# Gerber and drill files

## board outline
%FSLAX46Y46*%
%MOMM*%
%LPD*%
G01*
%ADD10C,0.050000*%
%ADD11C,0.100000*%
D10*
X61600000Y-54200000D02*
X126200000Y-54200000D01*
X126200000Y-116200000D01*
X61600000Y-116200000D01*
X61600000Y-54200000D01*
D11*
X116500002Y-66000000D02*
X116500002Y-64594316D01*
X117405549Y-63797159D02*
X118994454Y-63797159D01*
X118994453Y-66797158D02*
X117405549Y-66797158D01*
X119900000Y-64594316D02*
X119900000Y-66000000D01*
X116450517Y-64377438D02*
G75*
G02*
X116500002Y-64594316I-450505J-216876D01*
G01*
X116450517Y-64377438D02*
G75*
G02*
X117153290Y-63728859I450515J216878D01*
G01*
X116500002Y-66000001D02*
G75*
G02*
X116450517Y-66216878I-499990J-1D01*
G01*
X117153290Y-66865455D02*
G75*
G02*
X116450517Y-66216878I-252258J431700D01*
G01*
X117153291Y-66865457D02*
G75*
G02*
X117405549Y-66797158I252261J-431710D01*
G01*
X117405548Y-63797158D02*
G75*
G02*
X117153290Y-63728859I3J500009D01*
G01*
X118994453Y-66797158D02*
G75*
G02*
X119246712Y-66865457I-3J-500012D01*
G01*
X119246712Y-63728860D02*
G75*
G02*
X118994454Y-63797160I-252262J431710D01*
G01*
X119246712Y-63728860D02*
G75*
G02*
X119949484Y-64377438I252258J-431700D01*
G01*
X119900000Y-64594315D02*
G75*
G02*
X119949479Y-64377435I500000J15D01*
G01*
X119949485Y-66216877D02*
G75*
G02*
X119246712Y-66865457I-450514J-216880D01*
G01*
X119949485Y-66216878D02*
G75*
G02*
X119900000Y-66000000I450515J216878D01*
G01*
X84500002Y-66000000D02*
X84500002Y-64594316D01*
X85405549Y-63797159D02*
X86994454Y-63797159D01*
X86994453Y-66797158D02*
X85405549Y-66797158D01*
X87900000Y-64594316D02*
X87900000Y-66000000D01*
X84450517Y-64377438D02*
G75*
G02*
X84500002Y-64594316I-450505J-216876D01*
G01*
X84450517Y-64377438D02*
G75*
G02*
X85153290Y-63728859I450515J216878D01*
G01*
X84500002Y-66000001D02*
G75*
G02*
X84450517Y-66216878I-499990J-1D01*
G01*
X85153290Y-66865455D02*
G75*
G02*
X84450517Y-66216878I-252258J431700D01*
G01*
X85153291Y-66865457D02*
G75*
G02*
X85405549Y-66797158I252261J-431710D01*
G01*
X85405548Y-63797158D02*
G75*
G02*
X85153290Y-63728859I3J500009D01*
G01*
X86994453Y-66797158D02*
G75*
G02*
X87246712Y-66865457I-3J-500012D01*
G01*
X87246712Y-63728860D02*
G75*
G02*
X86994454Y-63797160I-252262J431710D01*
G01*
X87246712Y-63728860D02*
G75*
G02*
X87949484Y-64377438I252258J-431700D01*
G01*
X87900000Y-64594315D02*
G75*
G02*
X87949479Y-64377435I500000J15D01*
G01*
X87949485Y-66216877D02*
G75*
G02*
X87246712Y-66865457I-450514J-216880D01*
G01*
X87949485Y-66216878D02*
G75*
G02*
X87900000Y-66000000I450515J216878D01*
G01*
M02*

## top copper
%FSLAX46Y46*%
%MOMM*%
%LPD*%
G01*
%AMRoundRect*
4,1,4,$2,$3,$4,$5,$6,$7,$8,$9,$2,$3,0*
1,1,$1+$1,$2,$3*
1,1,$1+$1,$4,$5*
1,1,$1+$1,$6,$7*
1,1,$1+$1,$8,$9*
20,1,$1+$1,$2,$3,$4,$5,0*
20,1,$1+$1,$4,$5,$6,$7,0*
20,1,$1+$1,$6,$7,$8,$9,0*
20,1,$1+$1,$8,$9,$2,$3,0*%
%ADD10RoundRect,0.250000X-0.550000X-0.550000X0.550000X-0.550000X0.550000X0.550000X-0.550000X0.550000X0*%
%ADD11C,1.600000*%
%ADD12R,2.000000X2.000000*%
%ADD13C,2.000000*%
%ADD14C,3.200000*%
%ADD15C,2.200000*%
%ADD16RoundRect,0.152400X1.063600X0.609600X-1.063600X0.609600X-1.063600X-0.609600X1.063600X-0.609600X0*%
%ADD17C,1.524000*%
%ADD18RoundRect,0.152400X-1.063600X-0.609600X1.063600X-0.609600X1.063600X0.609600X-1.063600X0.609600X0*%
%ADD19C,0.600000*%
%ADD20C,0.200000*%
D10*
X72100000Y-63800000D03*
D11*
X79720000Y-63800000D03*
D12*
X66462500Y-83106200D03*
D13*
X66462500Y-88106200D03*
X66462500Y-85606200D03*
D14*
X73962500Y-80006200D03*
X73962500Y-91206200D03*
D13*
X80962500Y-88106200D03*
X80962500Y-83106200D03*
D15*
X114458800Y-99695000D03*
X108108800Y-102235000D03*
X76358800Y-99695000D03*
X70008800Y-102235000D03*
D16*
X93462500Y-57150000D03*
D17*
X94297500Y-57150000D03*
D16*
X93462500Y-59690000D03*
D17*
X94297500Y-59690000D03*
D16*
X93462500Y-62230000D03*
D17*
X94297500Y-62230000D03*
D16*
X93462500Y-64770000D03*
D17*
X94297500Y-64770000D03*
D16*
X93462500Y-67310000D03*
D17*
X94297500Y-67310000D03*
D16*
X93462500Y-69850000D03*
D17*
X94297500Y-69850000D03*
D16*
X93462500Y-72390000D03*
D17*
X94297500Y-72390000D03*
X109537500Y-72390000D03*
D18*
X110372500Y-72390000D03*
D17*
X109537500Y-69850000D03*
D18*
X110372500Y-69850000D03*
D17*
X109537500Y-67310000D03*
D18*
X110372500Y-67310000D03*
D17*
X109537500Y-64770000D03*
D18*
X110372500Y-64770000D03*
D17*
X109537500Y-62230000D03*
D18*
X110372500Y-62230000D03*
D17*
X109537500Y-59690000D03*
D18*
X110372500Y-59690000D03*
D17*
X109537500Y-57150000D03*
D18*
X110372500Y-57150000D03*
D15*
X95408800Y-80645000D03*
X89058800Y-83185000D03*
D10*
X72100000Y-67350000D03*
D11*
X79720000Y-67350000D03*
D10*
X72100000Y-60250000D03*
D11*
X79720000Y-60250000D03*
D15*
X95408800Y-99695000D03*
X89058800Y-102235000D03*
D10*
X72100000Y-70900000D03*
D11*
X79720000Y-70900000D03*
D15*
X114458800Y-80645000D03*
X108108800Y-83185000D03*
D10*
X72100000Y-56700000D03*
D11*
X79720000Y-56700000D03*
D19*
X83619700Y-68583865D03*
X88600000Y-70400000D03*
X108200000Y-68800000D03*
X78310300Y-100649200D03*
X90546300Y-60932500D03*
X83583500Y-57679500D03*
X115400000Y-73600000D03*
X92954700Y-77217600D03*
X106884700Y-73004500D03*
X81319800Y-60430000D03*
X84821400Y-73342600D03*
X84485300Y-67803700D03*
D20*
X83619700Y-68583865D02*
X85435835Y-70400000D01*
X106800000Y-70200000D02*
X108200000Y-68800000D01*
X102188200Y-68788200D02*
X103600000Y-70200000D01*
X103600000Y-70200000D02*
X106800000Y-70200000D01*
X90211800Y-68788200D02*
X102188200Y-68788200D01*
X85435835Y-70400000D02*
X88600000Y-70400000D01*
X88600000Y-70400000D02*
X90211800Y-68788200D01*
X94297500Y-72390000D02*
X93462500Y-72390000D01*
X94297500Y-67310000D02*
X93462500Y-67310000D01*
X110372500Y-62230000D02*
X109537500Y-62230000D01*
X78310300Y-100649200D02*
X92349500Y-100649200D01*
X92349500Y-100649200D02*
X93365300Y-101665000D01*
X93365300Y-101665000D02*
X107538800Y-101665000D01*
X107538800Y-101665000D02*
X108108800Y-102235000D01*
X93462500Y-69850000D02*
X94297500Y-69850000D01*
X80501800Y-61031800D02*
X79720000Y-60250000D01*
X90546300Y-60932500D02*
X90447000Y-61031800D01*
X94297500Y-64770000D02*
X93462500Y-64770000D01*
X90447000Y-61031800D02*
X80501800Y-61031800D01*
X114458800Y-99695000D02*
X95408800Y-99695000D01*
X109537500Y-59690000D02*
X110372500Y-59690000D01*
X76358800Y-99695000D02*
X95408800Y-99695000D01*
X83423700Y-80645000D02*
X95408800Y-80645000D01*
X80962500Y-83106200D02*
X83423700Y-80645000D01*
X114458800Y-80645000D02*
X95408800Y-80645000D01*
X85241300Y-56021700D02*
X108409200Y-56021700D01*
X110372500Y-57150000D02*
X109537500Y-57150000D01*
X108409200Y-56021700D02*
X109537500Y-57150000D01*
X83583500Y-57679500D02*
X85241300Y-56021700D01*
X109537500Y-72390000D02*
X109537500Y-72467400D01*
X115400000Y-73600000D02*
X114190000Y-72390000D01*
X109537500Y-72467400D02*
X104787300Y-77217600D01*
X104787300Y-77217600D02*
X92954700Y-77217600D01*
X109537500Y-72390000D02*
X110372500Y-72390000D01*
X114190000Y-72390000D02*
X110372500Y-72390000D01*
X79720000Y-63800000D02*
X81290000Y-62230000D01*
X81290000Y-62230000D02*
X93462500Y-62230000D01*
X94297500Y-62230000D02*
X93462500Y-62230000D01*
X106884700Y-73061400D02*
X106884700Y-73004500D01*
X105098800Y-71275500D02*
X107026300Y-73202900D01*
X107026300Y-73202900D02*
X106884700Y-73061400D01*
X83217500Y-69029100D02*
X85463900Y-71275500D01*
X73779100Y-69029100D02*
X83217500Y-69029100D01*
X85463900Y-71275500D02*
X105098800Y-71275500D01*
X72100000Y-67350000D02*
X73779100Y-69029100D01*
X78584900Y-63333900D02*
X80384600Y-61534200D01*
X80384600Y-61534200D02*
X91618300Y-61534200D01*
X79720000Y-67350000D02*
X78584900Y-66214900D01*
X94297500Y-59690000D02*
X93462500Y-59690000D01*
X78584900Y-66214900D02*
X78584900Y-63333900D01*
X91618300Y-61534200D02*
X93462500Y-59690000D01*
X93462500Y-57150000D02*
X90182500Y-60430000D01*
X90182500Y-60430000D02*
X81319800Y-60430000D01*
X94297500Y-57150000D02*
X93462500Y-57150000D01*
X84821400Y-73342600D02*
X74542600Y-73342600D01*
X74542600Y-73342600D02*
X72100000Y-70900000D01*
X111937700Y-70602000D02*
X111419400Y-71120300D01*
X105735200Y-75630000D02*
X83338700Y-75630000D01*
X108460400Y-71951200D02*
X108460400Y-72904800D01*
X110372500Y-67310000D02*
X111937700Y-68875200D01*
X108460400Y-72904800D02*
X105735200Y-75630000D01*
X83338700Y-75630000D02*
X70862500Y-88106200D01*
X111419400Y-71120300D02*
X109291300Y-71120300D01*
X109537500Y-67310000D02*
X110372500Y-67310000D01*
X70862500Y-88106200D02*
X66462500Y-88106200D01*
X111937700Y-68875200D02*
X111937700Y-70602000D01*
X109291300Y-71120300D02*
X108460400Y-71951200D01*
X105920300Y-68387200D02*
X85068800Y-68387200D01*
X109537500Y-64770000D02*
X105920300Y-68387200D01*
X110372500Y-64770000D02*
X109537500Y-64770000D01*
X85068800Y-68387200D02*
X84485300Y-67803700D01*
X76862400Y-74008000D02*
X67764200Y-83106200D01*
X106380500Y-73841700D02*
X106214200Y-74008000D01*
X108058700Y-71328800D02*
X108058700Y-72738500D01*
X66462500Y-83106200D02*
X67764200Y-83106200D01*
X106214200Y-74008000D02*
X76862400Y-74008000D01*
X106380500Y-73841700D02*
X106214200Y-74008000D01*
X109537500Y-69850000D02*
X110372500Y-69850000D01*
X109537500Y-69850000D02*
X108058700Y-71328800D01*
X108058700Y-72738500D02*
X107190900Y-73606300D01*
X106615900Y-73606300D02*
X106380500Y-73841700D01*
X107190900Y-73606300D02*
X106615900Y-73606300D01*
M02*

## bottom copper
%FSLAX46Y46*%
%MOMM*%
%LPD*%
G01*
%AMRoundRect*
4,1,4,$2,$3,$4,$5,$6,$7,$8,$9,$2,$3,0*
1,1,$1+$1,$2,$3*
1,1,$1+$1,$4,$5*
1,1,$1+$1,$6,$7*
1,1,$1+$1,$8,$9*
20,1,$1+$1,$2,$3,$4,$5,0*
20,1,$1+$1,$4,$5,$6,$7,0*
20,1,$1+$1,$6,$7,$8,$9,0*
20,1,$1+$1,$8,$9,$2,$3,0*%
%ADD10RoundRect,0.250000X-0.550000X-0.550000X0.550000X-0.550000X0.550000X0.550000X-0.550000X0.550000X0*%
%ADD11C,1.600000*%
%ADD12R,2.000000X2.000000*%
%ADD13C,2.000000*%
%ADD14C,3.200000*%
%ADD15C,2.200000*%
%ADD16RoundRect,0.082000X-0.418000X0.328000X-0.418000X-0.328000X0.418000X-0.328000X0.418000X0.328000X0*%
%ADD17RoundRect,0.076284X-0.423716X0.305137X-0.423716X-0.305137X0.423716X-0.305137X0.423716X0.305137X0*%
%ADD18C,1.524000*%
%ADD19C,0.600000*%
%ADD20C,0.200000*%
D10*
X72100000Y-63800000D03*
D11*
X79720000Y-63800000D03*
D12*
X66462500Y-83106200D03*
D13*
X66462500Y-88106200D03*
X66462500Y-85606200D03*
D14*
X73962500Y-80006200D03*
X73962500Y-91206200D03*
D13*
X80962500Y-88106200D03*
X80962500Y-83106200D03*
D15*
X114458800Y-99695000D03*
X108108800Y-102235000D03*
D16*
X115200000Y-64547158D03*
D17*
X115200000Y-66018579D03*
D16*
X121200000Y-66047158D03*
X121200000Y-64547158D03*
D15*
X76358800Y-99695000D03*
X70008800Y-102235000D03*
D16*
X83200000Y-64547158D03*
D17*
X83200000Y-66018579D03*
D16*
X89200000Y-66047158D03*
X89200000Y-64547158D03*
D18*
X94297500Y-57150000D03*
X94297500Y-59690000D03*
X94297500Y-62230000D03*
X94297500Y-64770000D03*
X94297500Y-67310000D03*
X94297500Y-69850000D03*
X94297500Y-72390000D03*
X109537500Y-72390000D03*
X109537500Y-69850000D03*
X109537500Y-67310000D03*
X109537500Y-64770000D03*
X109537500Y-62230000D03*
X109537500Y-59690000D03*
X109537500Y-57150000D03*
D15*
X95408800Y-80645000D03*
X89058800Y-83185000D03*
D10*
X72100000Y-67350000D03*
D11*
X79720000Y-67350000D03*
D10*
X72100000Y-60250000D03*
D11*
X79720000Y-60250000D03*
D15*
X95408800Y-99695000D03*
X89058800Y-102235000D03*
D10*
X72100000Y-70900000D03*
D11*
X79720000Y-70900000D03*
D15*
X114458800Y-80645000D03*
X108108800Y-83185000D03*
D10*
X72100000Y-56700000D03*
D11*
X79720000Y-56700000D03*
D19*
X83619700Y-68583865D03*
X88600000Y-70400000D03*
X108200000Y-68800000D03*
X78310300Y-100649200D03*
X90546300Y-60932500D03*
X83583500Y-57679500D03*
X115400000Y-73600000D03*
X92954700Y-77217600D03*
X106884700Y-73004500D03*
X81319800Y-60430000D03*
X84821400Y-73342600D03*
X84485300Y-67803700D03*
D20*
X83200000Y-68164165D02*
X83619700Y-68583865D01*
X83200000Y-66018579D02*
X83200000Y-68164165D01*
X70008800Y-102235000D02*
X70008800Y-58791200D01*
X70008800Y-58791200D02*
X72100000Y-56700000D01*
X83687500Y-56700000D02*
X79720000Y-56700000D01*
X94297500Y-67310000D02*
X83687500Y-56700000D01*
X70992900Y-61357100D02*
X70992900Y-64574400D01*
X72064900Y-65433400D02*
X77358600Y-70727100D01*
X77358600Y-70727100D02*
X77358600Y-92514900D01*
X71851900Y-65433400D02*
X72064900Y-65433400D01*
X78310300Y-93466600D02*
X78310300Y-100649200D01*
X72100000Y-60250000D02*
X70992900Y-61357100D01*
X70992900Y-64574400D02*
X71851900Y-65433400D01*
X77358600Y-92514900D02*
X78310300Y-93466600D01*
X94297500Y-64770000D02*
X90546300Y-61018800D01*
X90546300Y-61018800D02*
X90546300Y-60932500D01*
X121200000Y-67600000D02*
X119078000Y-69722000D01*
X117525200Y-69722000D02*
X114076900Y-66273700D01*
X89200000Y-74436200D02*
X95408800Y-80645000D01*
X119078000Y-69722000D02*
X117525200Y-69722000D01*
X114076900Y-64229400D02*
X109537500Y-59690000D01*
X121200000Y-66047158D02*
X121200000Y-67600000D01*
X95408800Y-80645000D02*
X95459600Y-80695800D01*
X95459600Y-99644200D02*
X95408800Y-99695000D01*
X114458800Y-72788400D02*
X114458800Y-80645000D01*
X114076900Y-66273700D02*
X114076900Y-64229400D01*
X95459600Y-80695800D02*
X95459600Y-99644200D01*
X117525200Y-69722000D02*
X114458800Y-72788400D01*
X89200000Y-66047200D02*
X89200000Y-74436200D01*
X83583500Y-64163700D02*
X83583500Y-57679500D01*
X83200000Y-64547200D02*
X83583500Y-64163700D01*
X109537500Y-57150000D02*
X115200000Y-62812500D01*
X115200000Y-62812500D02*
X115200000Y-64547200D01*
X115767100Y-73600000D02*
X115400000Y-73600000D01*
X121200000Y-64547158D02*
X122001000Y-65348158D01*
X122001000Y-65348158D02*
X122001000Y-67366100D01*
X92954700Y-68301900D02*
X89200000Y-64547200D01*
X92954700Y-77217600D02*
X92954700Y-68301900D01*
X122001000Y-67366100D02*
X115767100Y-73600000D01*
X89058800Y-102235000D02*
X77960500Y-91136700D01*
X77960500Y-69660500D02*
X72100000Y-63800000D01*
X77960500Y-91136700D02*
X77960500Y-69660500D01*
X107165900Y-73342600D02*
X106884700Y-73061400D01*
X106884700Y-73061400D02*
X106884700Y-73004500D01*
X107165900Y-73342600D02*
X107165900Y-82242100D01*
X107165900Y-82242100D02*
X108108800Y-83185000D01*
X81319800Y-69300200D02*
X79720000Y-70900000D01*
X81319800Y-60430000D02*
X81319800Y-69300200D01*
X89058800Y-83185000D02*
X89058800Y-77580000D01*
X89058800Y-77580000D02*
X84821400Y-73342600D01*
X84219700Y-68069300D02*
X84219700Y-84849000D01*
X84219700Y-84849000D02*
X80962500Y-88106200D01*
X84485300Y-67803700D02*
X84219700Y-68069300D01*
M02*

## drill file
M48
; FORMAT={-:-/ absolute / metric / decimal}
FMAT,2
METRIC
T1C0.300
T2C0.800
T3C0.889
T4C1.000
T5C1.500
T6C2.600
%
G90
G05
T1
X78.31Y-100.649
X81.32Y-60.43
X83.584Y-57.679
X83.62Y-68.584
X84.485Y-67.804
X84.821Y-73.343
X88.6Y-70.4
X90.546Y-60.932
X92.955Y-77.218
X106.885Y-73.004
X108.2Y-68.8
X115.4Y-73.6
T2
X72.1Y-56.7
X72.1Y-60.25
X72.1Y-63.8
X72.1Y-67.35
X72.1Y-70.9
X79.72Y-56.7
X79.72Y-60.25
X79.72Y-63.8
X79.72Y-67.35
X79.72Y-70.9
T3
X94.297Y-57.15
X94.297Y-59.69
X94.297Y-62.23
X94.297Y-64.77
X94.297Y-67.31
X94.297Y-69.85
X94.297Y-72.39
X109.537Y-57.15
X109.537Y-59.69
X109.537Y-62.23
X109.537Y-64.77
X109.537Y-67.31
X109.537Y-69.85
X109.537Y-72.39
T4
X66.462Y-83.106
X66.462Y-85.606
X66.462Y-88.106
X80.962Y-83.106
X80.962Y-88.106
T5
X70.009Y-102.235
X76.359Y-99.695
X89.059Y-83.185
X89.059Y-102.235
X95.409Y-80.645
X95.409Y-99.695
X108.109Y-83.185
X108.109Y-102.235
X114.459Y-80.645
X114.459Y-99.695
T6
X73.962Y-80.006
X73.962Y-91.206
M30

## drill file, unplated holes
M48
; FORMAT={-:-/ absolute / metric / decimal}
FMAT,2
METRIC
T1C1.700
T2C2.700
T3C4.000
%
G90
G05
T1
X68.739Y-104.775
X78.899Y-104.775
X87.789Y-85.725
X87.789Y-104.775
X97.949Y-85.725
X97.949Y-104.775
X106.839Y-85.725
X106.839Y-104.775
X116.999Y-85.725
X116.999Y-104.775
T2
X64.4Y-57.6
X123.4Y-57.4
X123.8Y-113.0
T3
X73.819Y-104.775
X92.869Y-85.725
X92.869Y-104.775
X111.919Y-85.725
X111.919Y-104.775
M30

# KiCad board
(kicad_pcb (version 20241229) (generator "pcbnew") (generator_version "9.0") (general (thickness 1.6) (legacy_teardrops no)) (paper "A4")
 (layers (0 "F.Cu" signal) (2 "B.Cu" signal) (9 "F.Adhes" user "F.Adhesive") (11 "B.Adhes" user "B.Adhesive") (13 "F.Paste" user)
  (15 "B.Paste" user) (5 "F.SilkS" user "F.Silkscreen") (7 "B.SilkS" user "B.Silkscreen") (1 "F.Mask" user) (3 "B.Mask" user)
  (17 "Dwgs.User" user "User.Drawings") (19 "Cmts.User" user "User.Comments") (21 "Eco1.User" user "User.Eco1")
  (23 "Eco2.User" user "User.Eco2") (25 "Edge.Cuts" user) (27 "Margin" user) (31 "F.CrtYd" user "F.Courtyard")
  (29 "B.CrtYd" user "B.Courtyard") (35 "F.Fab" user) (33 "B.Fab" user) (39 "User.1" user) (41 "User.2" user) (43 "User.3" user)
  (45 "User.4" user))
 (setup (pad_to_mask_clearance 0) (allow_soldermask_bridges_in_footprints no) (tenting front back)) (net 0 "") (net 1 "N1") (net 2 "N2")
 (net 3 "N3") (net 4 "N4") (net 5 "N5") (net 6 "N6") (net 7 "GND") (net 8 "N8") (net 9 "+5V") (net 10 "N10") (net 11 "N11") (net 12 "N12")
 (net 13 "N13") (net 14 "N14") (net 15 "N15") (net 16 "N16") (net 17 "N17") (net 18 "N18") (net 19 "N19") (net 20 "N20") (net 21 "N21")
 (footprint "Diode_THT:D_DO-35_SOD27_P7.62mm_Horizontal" (layer "F.Cu") (at 72.1 63.8)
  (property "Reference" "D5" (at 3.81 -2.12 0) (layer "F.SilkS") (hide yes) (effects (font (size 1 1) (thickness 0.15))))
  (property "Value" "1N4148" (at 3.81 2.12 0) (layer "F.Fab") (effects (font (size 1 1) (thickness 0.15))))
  (pad "1" thru_hole roundrect (at 0 0) (size 1.6 1.6) (drill 0.8) (layers "*.Cu" "*.Mask") (remove_unused_layers no)
   (roundrect_rratio 0.15625) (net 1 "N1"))
  (pad "2" thru_hole circle (at 7.62 0) (size 1.6 1.6) (drill 0.8) (layers "*.Cu" "*.Mask") (remove_unused_layers no) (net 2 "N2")))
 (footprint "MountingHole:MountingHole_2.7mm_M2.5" (layer "F.Cu") (at 123.4 57.4)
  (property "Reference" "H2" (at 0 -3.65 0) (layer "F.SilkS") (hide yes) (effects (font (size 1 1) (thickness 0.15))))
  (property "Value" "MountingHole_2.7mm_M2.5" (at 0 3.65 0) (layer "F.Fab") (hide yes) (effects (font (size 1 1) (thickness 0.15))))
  (pad "" np_thru_hole circle (at 0 0) (size 2.7 2.7) (drill 2.7) (layers "*.Cu" "*.Mask")))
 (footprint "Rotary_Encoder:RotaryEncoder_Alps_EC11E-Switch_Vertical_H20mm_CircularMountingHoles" (layer "F.Cu") (at 66.4625 83.1062)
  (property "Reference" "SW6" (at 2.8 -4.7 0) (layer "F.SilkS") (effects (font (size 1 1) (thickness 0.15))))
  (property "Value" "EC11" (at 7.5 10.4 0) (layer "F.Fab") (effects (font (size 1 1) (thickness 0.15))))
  (pad "A" thru_hole rect (at 0 0) (size 2 2) (drill 1) (layers "*.Cu" "*.Mask") (remove_unused_layers no) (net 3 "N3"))
  (pad "B" thru_hole circle (at 0 5) (size 2 2) (drill 1) (layers "*.Cu" "*.Mask") (remove_unused_layers no) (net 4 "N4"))
  (pad "C" thru_hole circle (at 0 2.5) (size 2 2) (drill 1) (layers "*.Cu" "*.Mask") (remove_unused_layers no) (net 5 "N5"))
  (pad "MP" thru_hole circle (at 7.5 -3.1) (size 3.2 3.2) (drill 2.6) (layers "*.Cu" "*.Mask") (remove_unused_layers no))
  (pad "MP" thru_hole circle (at 7.5 8.1) (size 3.2 3.2) (drill 2.6) (layers "*.Cu" "*.Mask") (remove_unused_layers no))
  (pad "S1" thru_hole circle (at 14.5 5) (size 2 2) (drill 1) (layers "*.Cu" "*.Mask") (remove_unused_layers no) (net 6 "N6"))
  (pad "S2" thru_hole circle (at 14.5 0) (size 2 2) (drill 1) (layers "*.Cu" "*.Mask") (remove_unused_layers no) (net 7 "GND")))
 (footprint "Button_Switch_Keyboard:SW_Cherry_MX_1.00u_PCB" (layer "F.Cu") (at 114.4588 99.695)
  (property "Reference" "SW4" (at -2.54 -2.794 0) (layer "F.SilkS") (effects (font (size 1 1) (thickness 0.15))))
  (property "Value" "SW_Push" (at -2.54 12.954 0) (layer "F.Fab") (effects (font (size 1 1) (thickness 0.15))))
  (pad "" np_thru_hole circle (at -7.62 5.08) (size 1.7 1.7) (drill 1.7) (layers "*.Cu" "*.Mask"))
  (pad "" np_thru_hole circle (at -2.54 5.08) (size 4 4) (drill 4) (layers "*.Cu" "*.Mask"))
  (pad "" np_thru_hole circle (at 2.54 5.08) (size 1.7 1.7) (drill 1.7) (layers "*.Cu" "*.Mask"))
  (pad "1" thru_hole circle (at 0 0) (size 2.2 2.2) (drill 1.5) (layers "*.Cu" "*.Mask") (remove_unused_layers no) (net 7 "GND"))
  (pad "2" thru_hole circle (at -6.35 2.54) (size 2.2 2.2) (drill 1.5) (layers "*.Cu" "*.Mask") (remove_unused_layers no) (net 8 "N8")))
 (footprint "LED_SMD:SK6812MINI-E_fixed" (layer "F.Cu") (at 118.2 65.4)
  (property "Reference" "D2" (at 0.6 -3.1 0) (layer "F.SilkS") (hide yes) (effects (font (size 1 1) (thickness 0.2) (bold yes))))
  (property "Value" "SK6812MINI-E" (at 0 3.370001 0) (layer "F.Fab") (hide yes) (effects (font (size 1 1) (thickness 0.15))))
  (fp_line (start -1.699998 0.6) (end -1.699998 -0.805684) (stroke (width 0.1) (type solid)) (layer "Edge.Cuts"))
  (fp_line (start -0.794451 -1.602841) (end 0.794454 -1.602841) (stroke (width 0.1) (type solid)) (layer "Edge.Cuts"))
  (fp_line (start 0.794453 1.397158) (end -0.794451 1.397158) (stroke (width 0.1) (type solid)) (layer "Edge.Cuts"))
  (fp_line (start 1.7 -0.805684) (end 1.7 0.6) (stroke (width 0.1) (type solid)) (layer "Edge.Cuts"))
  (fp_arc (start -1.749483 -1.022562) (mid -1.712526 -0.91691) (end -1.699998 -0.805684) (stroke (width 0.1) (type solid))
   (layer "Edge.Cuts"))
  (fp_arc (start -1.749483 -1.022562) (mid -1.63807 -1.606877) (end -1.04671 -1.671141) (stroke (width 0.1) (type solid))
   (layer "Edge.Cuts"))
  (fp_arc (start -1.699998 0.600001) (mid -1.712526 0.711226) (end -1.749483 0.816878) (stroke (width 0.1) (type solid)) (layer "Edge.Cuts"))
  (fp_arc (start -1.04671 1.465455) (mid -1.638069 1.401192) (end -1.749483 0.816878) (stroke (width 0.1) (type solid)) (layer "Edge.Cuts"))
  (fp_arc (start -1.046709 1.465457) (mid -0.925121 1.414535) (end -0.794451 1.397158) (stroke (width 0.1) (type solid)) (layer "Edge.Cuts"))
  (fp_arc (start -0.794452 -1.602842) (mid -0.925122 -1.620219) (end -1.04671 -1.671141) (stroke (width 0.1) (type solid))
   (layer "Edge.Cuts"))
  (fp_arc (start 0.794453 1.397158) (mid 0.925124 1.414535) (end 1.046712 1.465457) (stroke (width 0.1) (type solid)) (layer "Edge.Cuts"))
  (fp_arc (start 1.046712 -1.67114) (mid 0.925124 -1.620218) (end 0.794454 -1.602841) (stroke (width 0.1) (type solid)) (layer "Edge.Cuts"))
  (fp_arc (start 1.046712 -1.67114) (mid 1.638072 -1.606876) (end 1.749485 -1.022562) (stroke (width 0.1) (type solid)) (layer "Edge.Cuts"))
  (fp_arc (start 1.7 -0.805685) (mid 1.712528 -0.91691) (end 1.749485 -1.022562) (stroke (width 0.1) (type solid)) (layer "Edge.Cuts"))
  (fp_arc (start 1.749485 0.816877) (mid 1.638073 1.401193) (end 1.046712 1.465457) (stroke (width 0.1) (type solid)) (layer "Edge.Cuts"))
  (fp_arc (start 1.749485 0.816878) (mid 1.712528 0.711226) (end 1.7 0.6) (stroke (width 0.1) (type solid)) (layer "Edge.Cuts"))
  (pad "1" smd roundrect (at -3 -0.852842 270) (size 0.82 1) (layers "B.Cu" "B.Mask" "B.Paste") (roundrect_rratio 0.1) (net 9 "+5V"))
  (pad "2" smd roundrect (at -3 0.618579 270) (size 0.762842 1) (layers "B.Cu" "B.Mask" "B.Paste") (roundrect_rratio 0.1) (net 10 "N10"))
  (pad "3" smd roundrect (at 3 0.647158 270) (size 0.82 1) (layers "B.Cu" "B.Mask" "B.Paste") (roundrect_rratio 0.1) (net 7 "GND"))
  (pad "4" smd roundrect (at 3 -0.852842 270) (size 0.82 1) (layers "B.Cu" "B.Mask" "B.Paste") (roundrect_rratio 0.1) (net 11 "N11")))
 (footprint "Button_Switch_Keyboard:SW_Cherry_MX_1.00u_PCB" (layer "F.Cu") (at 76.3588 99.695)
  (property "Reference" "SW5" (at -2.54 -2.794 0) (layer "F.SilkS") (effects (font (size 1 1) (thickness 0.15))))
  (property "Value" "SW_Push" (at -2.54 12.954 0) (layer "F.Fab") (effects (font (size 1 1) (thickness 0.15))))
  (pad "" np_thru_hole circle (at -7.62 5.08) (size 1.7 1.7) (drill 1.7) (layers "*.Cu" "*.Mask"))
  (pad "" np_thru_hole circle (at -2.54 5.08) (size 4 4) (drill 4) (layers "*.Cu" "*.Mask"))
  (pad "" np_thru_hole circle (at 2.54 5.08) (size 1.7 1.7) (drill 1.7) (layers "*.Cu" "*.Mask"))
  (pad "1" thru_hole circle (at 0 0) (size 2.2 2.2) (drill 1.5) (layers "*.Cu" "*.Mask") (remove_unused_layers no) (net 7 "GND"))
  (pad "2" thru_hole circle (at -6.35 2.54) (size 2.2 2.2) (drill 1.5) (layers "*.Cu" "*.Mask") (remove_unused_layers no) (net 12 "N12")))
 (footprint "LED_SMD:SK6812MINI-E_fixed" (layer "F.Cu") (at 86.2 65.4)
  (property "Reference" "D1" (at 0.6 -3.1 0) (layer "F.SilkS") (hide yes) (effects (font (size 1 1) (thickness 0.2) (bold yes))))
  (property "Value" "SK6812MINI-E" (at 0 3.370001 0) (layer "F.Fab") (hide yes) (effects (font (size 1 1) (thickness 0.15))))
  (fp_line (start -1.699998 0.6) (end -1.699998 -0.805684) (stroke (width 0.1) (type solid)) (layer "Edge.Cuts"))
  (fp_line (start -0.794451 -1.602841) (end 0.794454 -1.602841) (stroke (width 0.1) (type solid)) (layer "Edge.Cuts"))
  (fp_line (start 0.794453 1.397158) (end -0.794451 1.397158) (stroke (width 0.1) (type solid)) (layer "Edge.Cuts"))
  (fp_line (start 1.7 -0.805684) (end 1.7 0.6) (stroke (width 0.1) (type solid)) (layer "Edge.Cuts"))
  (fp_arc (start -1.749483 -1.022562) (mid -1.712526 -0.91691) (end -1.699998 -0.805684) (stroke (width 0.1) (type solid))
   (layer "Edge.Cuts"))
  (fp_arc (start -1.749483 -1.022562) (mid -1.63807 -1.606877) (end -1.04671 -1.671141) (stroke (width 0.1) (type solid))
   (layer "Edge.Cuts"))
  (fp_arc (start -1.699998 0.600001) (mid -1.712526 0.711226) (end -1.749483 0.816878) (stroke (width 0.1) (type solid)) (layer "Edge.Cuts"))
  (fp_arc (start -1.04671 1.465455) (mid -1.638069 1.401192) (end -1.749483 0.816878) (stroke (width 0.1) (type solid)) (layer "Edge.Cuts"))
  (fp_arc (start -1.046709 1.465457) (mid -0.925121 1.414535) (end -0.794451 1.397158) (stroke (width 0.1) (type solid)) (layer "Edge.Cuts"))
  (fp_arc (start -0.794452 -1.602842) (mid -0.925122 -1.620219) (end -1.04671 -1.671141) (stroke (width 0.1) (type solid))
   (layer "Edge.Cuts"))
  (fp_arc (start 0.794453 1.397158) (mid 0.925124 1.414535) (end 1.046712 1.465457) (stroke (width 0.1) (type solid)) (layer "Edge.Cuts"))
  (fp_arc (start 1.046712 -1.67114) (mid 0.925124 -1.620218) (end 0.794454 -1.602841) (stroke (width 0.1) (type solid)) (layer "Edge.Cuts"))
  (fp_arc (start 1.046712 -1.67114) (mid 1.638072 -1.606876) (end 1.749485 -1.022562) (stroke (width 0.1) (type solid)) (layer "Edge.Cuts"))
  (fp_arc (start 1.7 -0.805685) (mid 1.712528 -0.91691) (end 1.749485 -1.022562) (stroke (width 0.1) (type solid)) (layer "Edge.Cuts"))
  (fp_arc (start 1.749485 0.816877) (mid 1.638073 1.401193) (end 1.046712 1.465457) (stroke (width 0.1) (type solid)) (layer "Edge.Cuts"))
  (fp_arc (start 1.749485 0.816878) (mid 1.712528 0.711226) (end 1.7 0.6) (stroke (width 0.1) (type solid)) (layer "Edge.Cuts"))
  (pad "1" smd roundrect (at -3 -0.852842 270) (size 0.82 1) (layers "B.Cu" "B.Mask" "B.Paste") (roundrect_rratio 0.1) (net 9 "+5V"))
  (pad "2" smd roundrect (at -3 0.618579 270) (size 0.762842 1) (layers "B.Cu" "B.Mask" "B.Paste") (roundrect_rratio 0.1))
  (pad "3" smd roundrect (at 3 0.647158 270) (size 0.82 1) (layers "B.Cu" "B.Mask" "B.Paste") (roundrect_rratio 0.1) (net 7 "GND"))
  (pad "4" smd roundrect (at 3 -0.852842 270) (size 0.82 1) (layers "B.Cu" "B.Mask" "B.Paste") (roundrect_rratio 0.1) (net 11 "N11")))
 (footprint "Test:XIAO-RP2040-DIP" (layer "F.Cu") (at 101.9175 64.77)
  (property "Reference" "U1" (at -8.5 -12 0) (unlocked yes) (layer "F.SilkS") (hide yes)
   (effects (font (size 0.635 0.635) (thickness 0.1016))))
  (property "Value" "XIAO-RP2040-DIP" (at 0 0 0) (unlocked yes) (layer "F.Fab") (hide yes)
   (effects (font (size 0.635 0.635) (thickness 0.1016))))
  (pad "1" smd roundrect (at -8.455 -7.62 180) (size 2.432 1.524) (layers "F.Cu" "F.Mask") (roundrect_rratio 0.1) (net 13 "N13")
   (thermal_bridge_angle 45))
  (pad "1" thru_hole circle (at -7.62 -7.62 180) (size 1.524 1.524) (drill 0.889) (layers "*.Cu" "*.Mask") (remove_unused_layers no)
   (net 13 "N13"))
  (pad "2" smd roundrect (at -8.455 -5.08 180) (size 2.432 1.524) (layers "F.Cu" "F.Mask") (roundrect_rratio 0.1) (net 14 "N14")
   (thermal_bridge_angle 45))
  (pad "2" thru_hole circle (at -7.62 -5.08 180) (size 1.524 1.524) (drill 0.889) (layers "*.Cu" "*.Mask") (remove_unused_layers no)
   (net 14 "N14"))
  (pad "3" smd roundrect (at -8.455 -2.54 180) (size 2.432 1.524) (layers "F.Cu" "F.Mask") (roundrect_rratio 0.1) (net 2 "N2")
   (thermal_bridge_angle 45))
  (pad "3" thru_hole circle (at -7.62 -2.54 180) (size 1.524 1.524) (drill 0.889) (layers "*.Cu" "*.Mask") (remove_unused_layers no)
   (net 2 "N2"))
  (pad "4" smd roundrect (at -8.455 0 180) (size 2.432 1.524) (layers "F.Cu" "F.Mask") (roundrect_rratio 0.1) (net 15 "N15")
   (thermal_bridge_angle 45))
  (pad "4" thru_hole circle (at -7.62 0 180) (size 1.524 1.524) (drill 0.889) (layers "*.Cu" "*.Mask") (remove_unused_layers no)
   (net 15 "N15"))
  (pad "5" smd roundrect (at -8.455 2.54 180) (size 2.432 1.524) (layers "F.Cu" "F.Mask") (roundrect_rratio 0.1) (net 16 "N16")
   (thermal_bridge_angle 45))
  (pad "5" thru_hole circle (at -7.62 2.54 180) (size 1.524 1.524) (drill 0.889) (layers "*.Cu" "*.Mask") (remove_unused_layers no)
   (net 16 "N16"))
  (pad "6" smd roundrect (at -8.455 5.08 180) (size 2.432 1.524) (layers "F.Cu" "F.Mask") (roundrect_rratio 0.1) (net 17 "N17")
   (thermal_bridge_angle 45))
  (pad "6" thru_hole circle (at -7.62 5.08 180) (size 1.524 1.524) (drill 0.889) (layers "*.Cu" "*.Mask") (remove_unused_layers no)
   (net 17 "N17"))
  (pad "7" smd roundrect (at -8.455 7.62 180) (size 2.432 1.524) (layers "F.Cu" "F.Mask") (roundrect_rratio 0.1) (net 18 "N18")
   (thermal_bridge_angle 45))
  (pad "7" thru_hole circle (at -7.62 7.62 180) (size 1.524 1.524) (drill 0.889) (layers "*.Cu" "*.Mask") (remove_unused_layers no)
   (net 18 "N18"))
  (pad "8" thru_hole circle (at 7.62 7.62) (size 1.524 1.524) (drill 0.889) (layers "*.Cu" "*.Mask") (remove_unused_layers no)
   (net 11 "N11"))
  (pad "8" smd roundrect (at 8.455 7.62) (size 2.432 1.524) (layers "F.Cu" "F.Mask") (roundrect_rratio 0.1) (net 11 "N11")
   (thermal_bridge_angle 45))
  (pad "9" thru_hole circle (at 7.62 5.08) (size 1.524 1.524) (drill 0.889) (layers "*.Cu" "*.Mask") (remove_unused_layers no) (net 3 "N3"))
  (pad "9" smd roundrect (at 8.455 5.08) (size 2.432 1.524) (layers "F.Cu" "F.Mask") (roundrect_rratio 0.1) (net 3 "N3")
   (thermal_bridge_angle 45))
  (pad "10" thru_hole circle (at 7.62 2.54) (size 1.524 1.524) (drill 0.889) (layers "*.Cu" "*.Mask") (remove_unused_layers no) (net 4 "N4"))
  (pad "10" smd roundrect (at 8.455 2.54) (size 2.432 1.524) (layers "F.Cu" "F.Mask") (roundrect_rratio 0.1) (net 4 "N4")
   (thermal_bridge_angle 45))
  (pad "11" thru_hole circle (at 7.62 0) (size 1.524 1.524) (drill 0.889) (layers "*.Cu" "*.Mask") (remove_unused_layers no) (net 6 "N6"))
  (pad "11" smd roundrect (at 8.455 0) (size 2.432 1.524) (layers "F.Cu" "F.Mask") (roundrect_rratio 0.1) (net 6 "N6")
   (thermal_bridge_angle 45))
  (pad "12" thru_hole circle (at 7.62 -2.54) (size 1.524 1.524) (drill 0.889) (layers "*.Cu" "*.Mask") (remove_unused_layers no)
   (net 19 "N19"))
  (pad "12" smd roundrect (at 8.455 -2.54) (size 2.432 1.524) (layers "F.Cu" "F.Mask") (roundrect_rratio 0.1) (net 19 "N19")
   (thermal_bridge_angle 45))
  (pad "13" thru_hole circle (at 7.62 -5.08) (size 1.524 1.524) (drill 0.889) (layers "*.Cu" "*.Mask") (remove_unused_layers no)
   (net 7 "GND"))
  (pad "13" smd roundrect (at 8.455 -5.08) (size 2.432 1.524) (layers "F.Cu" "F.Mask") (roundrect_rratio 0.1) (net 7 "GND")
   (thermal_bridge_angle 45))
  (pad "14" thru_hole circle (at 7.62 -7.62) (size 1.524 1.524) (drill 0.889) (layers "*.Cu" "*.Mask") (remove_unused_layers no)
   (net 9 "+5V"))
  (pad "14" smd roundrect (at 8.455 -7.62) (size 2.432 1.524) (layers "F.Cu" "F.Mask") (roundrect_rratio 0.1) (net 9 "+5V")
   (thermal_bridge_angle 45)))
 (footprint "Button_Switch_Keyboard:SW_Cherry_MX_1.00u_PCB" (layer "F.Cu") (at 95.4088 80.645)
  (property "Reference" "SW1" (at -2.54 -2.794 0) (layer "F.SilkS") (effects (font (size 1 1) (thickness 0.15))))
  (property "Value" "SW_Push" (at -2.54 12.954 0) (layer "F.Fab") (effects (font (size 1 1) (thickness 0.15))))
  (pad "" np_thru_hole circle (at -7.62 5.08) (size 1.7 1.7) (drill 1.7) (layers "*.Cu" "*.Mask"))
  (pad "" np_thru_hole circle (at -2.54 5.08) (size 4 4) (drill 4) (layers "*.Cu" "*.Mask"))
  (pad "" np_thru_hole circle (at 2.54 5.08) (size 1.7 1.7) (drill 1.7) (layers "*.Cu" "*.Mask"))
  (pad "1" thru_hole circle (at 0 0) (size 2.2 2.2) (drill 1.5) (layers "*.Cu" "*.Mask") (remove_unused_layers no) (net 7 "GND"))
  (pad "2" thru_hole circle (at -6.35 2.54) (size 2.2 2.2) (drill 1.5) (layers "*.Cu" "*.Mask") (remove_unused_layers no) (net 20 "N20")))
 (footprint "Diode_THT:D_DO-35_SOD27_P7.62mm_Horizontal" (layer "F.Cu") (at 72.1 67.35)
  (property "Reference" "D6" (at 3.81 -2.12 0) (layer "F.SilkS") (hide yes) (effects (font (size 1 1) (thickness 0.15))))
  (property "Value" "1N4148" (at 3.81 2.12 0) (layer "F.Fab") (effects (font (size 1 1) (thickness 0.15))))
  (pad "1" thru_hole roundrect (at 0 0) (size 1.6 1.6) (drill 0.8) (layers "*.Cu" "*.Mask") (remove_unused_layers no)
   (roundrect_rratio 0.15625) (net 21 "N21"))
  (pad "2" thru_hole circle (at 7.62 0) (size 1.6 1.6) (drill 0.8) (layers "*.Cu" "*.Mask") (remove_unused_layers no) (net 14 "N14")))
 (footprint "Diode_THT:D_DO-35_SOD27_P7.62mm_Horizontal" (layer "F.Cu") (at 72.1 60.25)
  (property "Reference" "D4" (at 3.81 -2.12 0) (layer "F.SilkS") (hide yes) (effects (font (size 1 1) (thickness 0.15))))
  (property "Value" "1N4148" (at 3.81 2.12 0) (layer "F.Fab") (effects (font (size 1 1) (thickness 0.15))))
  (pad "1" thru_hole roundrect (at 0 0) (size 1.6 1.6) (drill 0.8) (layers "*.Cu" "*.Mask") (remove_unused_layers no)
   (roundrect_rratio 0.15625) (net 8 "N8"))
  (pad "2" thru_hole circle (at 7.62 0) (size 1.6 1.6) (drill 0.8) (layers "*.Cu" "*.Mask") (remove_unused_layers no) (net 15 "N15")))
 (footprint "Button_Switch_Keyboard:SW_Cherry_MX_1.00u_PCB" (layer "F.Cu") (at 95.4088 99.695)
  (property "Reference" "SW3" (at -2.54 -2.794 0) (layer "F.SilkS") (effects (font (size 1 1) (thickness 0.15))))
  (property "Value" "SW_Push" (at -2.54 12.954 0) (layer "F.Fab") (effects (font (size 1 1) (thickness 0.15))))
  (pad "" np_thru_hole circle (at -7.62 5.08) (size 1.7 1.7) (drill 1.7) (layers "*.Cu" "*.Mask"))
  (pad "" np_thru_hole circle (at -2.54 5.08) (size 4 4) (drill 4) (layers "*.Cu" "*.Mask"))
  (pad "" np_thru_hole circle (at 2.54 5.08) (size 1.7 1.7) (drill 1.7) (layers "*.Cu" "*.Mask"))
  (pad "1" thru_hole circle (at 0 0) (size 2.2 2.2) (drill 1.5) (layers "*.Cu" "*.Mask") (remove_unused_layers no) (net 7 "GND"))
  (pad "2" thru_hole circle (at -6.35 2.54) (size 2.2 2.2) (drill 1.5) (layers "*.Cu" "*.Mask") (remove_unused_layers no) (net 1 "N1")))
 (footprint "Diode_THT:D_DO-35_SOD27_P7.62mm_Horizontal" (layer "F.Cu") (at 72.1 70.9)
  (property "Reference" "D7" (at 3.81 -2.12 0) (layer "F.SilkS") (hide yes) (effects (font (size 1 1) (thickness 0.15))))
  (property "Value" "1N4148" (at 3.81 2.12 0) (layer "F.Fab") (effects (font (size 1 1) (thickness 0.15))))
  (pad "1" thru_hole roundrect (at 0 0) (size 1.6 1.6) (drill 0.8) (layers "*.Cu" "*.Mask") (remove_unused_layers no)
   (roundrect_rratio 0.15625) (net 20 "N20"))
  (pad "2" thru_hole circle (at 7.62 0) (size 1.6 1.6) (drill 0.8) (layers "*.Cu" "*.Mask") (remove_unused_layers no) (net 13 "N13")))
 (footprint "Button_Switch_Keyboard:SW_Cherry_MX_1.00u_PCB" (layer "F.Cu") (at 114.4588 80.645)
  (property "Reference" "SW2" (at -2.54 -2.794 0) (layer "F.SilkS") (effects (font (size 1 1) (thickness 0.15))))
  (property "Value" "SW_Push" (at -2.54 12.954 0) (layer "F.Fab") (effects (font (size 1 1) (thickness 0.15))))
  (pad "" np_thru_hole circle (at -7.62 5.08) (size 1.7 1.7) (drill 1.7) (layers "*.Cu" "*.Mask"))
  (pad "" np_thru_hole circle (at -2.54 5.08) (size 4 4) (drill 4) (layers "*.Cu" "*.Mask"))
  (pad "" np_thru_hole circle (at 2.54 5.08) (size 1.7 1.7) (drill 1.7) (layers "*.Cu" "*.Mask"))
  (pad "1" thru_hole circle (at 0 0) (size 2.2 2.2) (drill 1.5) (layers "*.Cu" "*.Mask") (remove_unused_layers no) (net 7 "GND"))
  (pad "2" thru_hole circle (at -6.35 2.54) (size 2.2 2.2) (drill 1.5) (layers "*.Cu" "*.Mask") (remove_unused_layers no) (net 21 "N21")))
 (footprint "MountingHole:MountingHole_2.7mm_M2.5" (layer "F.Cu") (at 64.4 57.6)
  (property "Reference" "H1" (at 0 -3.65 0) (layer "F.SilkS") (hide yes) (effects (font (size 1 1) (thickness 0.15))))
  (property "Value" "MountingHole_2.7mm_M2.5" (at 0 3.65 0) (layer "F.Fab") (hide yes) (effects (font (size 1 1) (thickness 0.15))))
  (pad "" np_thru_hole circle (at 0 0) (size 2.7 2.7) (drill 2.7) (layers "*.Cu" "*.Mask")))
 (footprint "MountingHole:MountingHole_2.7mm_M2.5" (layer "F.Cu") (at 123.8 113)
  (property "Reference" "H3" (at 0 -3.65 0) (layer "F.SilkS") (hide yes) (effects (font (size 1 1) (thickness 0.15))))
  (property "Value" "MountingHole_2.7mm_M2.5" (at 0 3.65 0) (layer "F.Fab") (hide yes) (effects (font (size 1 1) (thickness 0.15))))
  (pad "" np_thru_hole circle (at 0 0) (size 2.7 2.7) (drill 2.7) (layers "*.Cu" "*.Mask")))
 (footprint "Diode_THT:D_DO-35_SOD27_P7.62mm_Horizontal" (layer "F.Cu") (at 72.1 56.7)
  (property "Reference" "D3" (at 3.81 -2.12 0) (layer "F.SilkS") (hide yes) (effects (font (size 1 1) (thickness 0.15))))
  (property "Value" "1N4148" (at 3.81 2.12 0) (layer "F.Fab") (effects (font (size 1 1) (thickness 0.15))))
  (pad "1" thru_hole roundrect (at 0 0) (size 1.6 1.6) (drill 0.8) (layers "*.Cu" "*.Mask") (remove_unused_layers no)
   (roundrect_rratio 0.15625) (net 12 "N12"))
  (pad "2" thru_hole circle (at 7.62 0) (size 1.6 1.6) (drill 0.8) (layers "*.Cu" "*.Mask") (remove_unused_layers no) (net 16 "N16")))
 (gr_rect (start 61.6 54.2) (end 126.2 116.2) (stroke (width 0.05) (type default)) (fill no) (layer "Edge.Cuts"))
 (segment (start 83.6197 68.583865) (end 85.435835 70.4) (width 0.2) (layer "F.Cu") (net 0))
 (segment (start 106.8 70.2) (end 108.2 68.8) (width 0.2) (layer "F.Cu") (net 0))
 (segment (start 102.1882 68.7882) (end 103.6 70.2) (width 0.2) (layer "F.Cu") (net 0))
 (segment (start 103.6 70.2) (end 106.8 70.2) (width 0.2) (layer "F.Cu") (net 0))
 (segment (start 90.2118 68.7882) (end 102.1882 68.7882) (width 0.2) (layer "F.Cu") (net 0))
 (segment (start 85.435835 70.4) (end 88.6 70.4) (width 0.2) (layer "F.Cu") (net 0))
 (segment (start 88.6 70.4) (end 90.2118 68.7882) (width 0.2) (layer "F.Cu") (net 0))
 (via (at 83.6197 68.583865) (size 0.6) (drill 0.3) (layers "F.Cu" "B.Cu") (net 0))
 (via (at 88.6 70.4) (size 0.6) (drill 0.3) (layers "F.Cu" "B.Cu") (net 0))
 (via (at 108.2 68.8) (size 0.6) (drill 0.3) (layers "F.Cu" "B.Cu") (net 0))
 (segment (start 83.2 68.164165) (end 83.6197 68.583865) (width 0.2) (layer "B.Cu") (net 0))
 (segment (start 83.2 66.018579) (end 83.2 68.164165) (width 0.2) (layer "B.Cu") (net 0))
 (segment (start 94.2975 72.39) (end 93.4625 72.39) (width 0.2) (layer "F.Cu") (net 18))
 (segment (start 70.0088 102.235) (end 70.0088 58.7912) (width 0.2) (layer "B.Cu") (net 12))
 (segment (start 70.0088 58.7912) (end 72.1 56.7) (width 0.2) (layer "B.Cu") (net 12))
 (segment (start 94.2975 67.31) (end 93.4625 67.31) (width 0.2) (layer "F.Cu") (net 16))
 (segment (start 83.6875 56.7) (end 79.72 56.7) (width 0.2) (layer "B.Cu") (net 16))
 (segment (start 94.2975 67.31) (end 83.6875 56.7) (width 0.2) (layer "B.Cu") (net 16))
 (segment (start 110.3725 62.23) (end 109.5375 62.23) (width 0.2) (layer "F.Cu") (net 19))
 (segment (start 78.3103 100.6492) (end 92.3495 100.6492) (width 0.2) (layer "F.Cu") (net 8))
 (segment (start 92.3495 100.6492) (end 93.3653 101.665) (width 0.2) (layer "F.Cu") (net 8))
 (segment (start 93.3653 101.665) (end 107.5388 101.665) (width 0.2) (layer "F.Cu") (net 8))
 (segment (start 107.5388 101.665) (end 108.1088 102.235) (width 0.2) (layer "F.Cu") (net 8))
 (via (at 78.3103 100.6492) (size 0.6) (drill 0.3) (layers "F.Cu" "B.Cu") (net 8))
 (segment (start 70.9929 61.3571) (end 70.9929 64.5744) (width 0.2) (layer "B.Cu") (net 8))
 (segment (start 72.0649 65.4334) (end 77.3586 70.7271) (width 0.2) (layer "B.Cu") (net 8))
 (segment (start 77.3586 70.7271) (end 77.3586 92.5149) (width 0.2) (layer "B.Cu") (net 8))
 (segment (start 71.8519 65.4334) (end 72.0649 65.4334) (width 0.2) (layer "B.Cu") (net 8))
 (segment (start 78.3103 93.4666) (end 78.3103 100.6492) (width 0.2) (layer "B.Cu") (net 8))
 (segment (start 72.1 60.25) (end 70.9929 61.3571) (width 0.2) (layer "B.Cu") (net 8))
 (segment (start 70.9929 64.5744) (end 71.8519 65.4334) (width 0.2) (layer "B.Cu") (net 8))
 (segment (start 77.3586 92.5149) (end 78.3103 93.4666) (width 0.2) (layer "B.Cu") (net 8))
 (segment (start 93.4625 69.85) (end 94.2975 69.85) (width 0.2) (layer "F.Cu") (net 17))
 (segment (start 80.5018 61.0318) (end 79.72 60.25) (width 0.2) (layer "F.Cu") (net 15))
 (segment (start 90.5463 60.9325) (end 90.447 61.0318) (width 0.2) (layer "F.Cu") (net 15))
 (segment (start 94.2975 64.77) (end 93.4625 64.77) (width 0.2) (layer "F.Cu") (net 15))
 (segment (start 90.447 61.0318) (end 80.5018 61.0318) (width 0.2) (layer "F.Cu") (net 15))
 (via (at 90.5463 60.9325) (size 0.6) (drill 0.3) (layers "F.Cu" "B.Cu") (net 15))
 (segment (start 94.2975 64.77) (end 90.5463 61.0188) (width 0.2) (layer "B.Cu") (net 15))
 (segment (start 90.5463 61.0188) (end 90.5463 60.9325) (width 0.2) (layer "B.Cu") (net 15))
 (segment (start 114.4588 99.695) (end 95.4088 99.695) (width 0.2) (layer "F.Cu") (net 7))
 (segment (start 109.5375 59.69) (end 110.3725 59.69) (width 0.2) (layer "F.Cu") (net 7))
 (segment (start 76.3588 99.695) (end 95.4088 99.695) (width 0.2) (layer "F.Cu") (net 7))
 (segment (start 83.4237 80.645) (end 95.4088 80.645) (width 0.2) (layer "F.Cu") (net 7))
 (segment (start 80.9625 83.1062) (end 83.4237 80.645) (width 0.2) (layer "F.Cu") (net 7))
 (segment (start 114.4588 80.645) (end 95.4088 80.645) (width 0.2) (layer "F.Cu") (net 7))
 (segment (start 121.2 67.6) (end 119.078 69.722) (width 0.2) (layer "B.Cu") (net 7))
 (segment (start 117.5252 69.722) (end 114.0769 66.2737) (width 0.2) (layer "B.Cu") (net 7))
 (segment (start 89.2 74.4362) (end 95.4088 80.645) (width 0.2) (layer "B.Cu") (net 7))
 (segment (start 119.078 69.722) (end 117.5252 69.722) (width 0.2) (layer "B.Cu") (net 7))
 (segment (start 114.0769 64.2294) (end 109.5375 59.69) (width 0.2) (layer "B.Cu") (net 7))
 (segment (start 121.2 66.047158) (end 121.2 67.6) (width 0.2) (layer "B.Cu") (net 7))
 (segment (start 95.4088 80.645) (end 95.4596 80.6958) (width 0.2) (layer "B.Cu") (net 7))
 (segment (start 95.4596 99.6442) (end 95.4088 99.695) (width 0.2) (layer "B.Cu") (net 7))
 (segment (start 114.4588 72.7884) (end 114.4588 80.645) (width 0.2) (layer "B.Cu") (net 7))
 (segment (start 114.0769 66.2737) (end 114.0769 64.2294) (width 0.2) (layer "B.Cu") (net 7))
 (segment (start 95.4596 80.6958) (end 95.4596 99.6442) (width 0.2) (layer "B.Cu") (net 7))
 (segment (start 117.5252 69.722) (end 114.4588 72.7884) (width 0.2) (layer "B.Cu") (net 7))
 (segment (start 89.2 66.0472) (end 89.2 74.4362) (width 0.2) (layer "B.Cu") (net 7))
 (segment (start 85.2413 56.0217) (end 108.4092 56.0217) (width 0.2) (layer "F.Cu") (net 9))
 (segment (start 110.3725 57.15) (end 109.5375 57.15) (width 0.2) (layer "F.Cu") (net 9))
 (segment (start 108.4092 56.0217) (end 109.5375 57.15) (width 0.2) (layer "F.Cu") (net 9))
 (segment (start 83.5835 57.6795) (end 85.2413 56.0217) (width 0.2) (layer "F.Cu") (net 9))
 (via (at 83.5835 57.6795) (size 0.6) (drill 0.3) (layers "F.Cu" "B.Cu") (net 9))
 (segment (start 83.5835 64.1637) (end 83.5835 57.6795) (width 0.2) (layer "B.Cu") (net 9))
 (segment (start 83.2 64.5472) (end 83.5835 64.1637) (width 0.2) (layer "B.Cu") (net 9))
 (segment (start 109.5375 57.15) (end 115.2 62.8125) (width 0.2) (layer "B.Cu") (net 9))
 (segment (start 115.2 62.8125) (end 115.2 64.5472) (width 0.2) (layer "B.Cu") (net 9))
 (segment (start 109.5375 72.39) (end 109.5375 72.4674) (width 0.2) (layer "F.Cu") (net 11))
 (segment (start 115.4 73.6) (end 114.19 72.39) (width 0.2) (layer "F.Cu") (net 11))
 (segment (start 109.5375 72.4674) (end 104.7873 77.2176) (width 0.2) (layer "F.Cu") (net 11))
 (segment (start 104.7873 77.2176) (end 92.9547 77.2176) (width 0.2) (layer "F.Cu") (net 11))
 (segment (start 109.5375 72.39) (end 110.3725 72.39) (width 0.2) (layer "F.Cu") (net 11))
 (segment (start 114.19 72.39) (end 110.3725 72.39) (width 0.2) (layer "F.Cu") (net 11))
 (via (at 115.4 73.6) (size 0.6) (drill 0.3) (layers "F.Cu" "B.Cu") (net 11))
 (via (at 92.9547 77.2176) (size 0.6) (drill 0.3) (layers "F.Cu" "B.Cu") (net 11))
 (segment (start 115.7671 73.6) (end 115.4 73.6) (width 0.2) (layer "B.Cu") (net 11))
 (segment (start 121.2 64.547158) (end 122.001 65.348158) (width 0.2) (layer "B.Cu") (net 11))
 (segment (start 122.001 65.348158) (end 122.001 67.3661) (width 0.2) (layer "B.Cu") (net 11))
 (segment (start 92.9547 68.3019) (end 89.2 64.5472) (width 0.2) (layer "B.Cu") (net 11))
 (segment (start 92.9547 77.2176) (end 92.9547 68.3019) (width 0.2) (layer "B.Cu") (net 11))
 (segment (start 122.001 67.3661) (end 115.7671 73.6) (width 0.2) (layer "B.Cu") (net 11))
 (segment (start 89.0588 102.235) (end 77.9605 91.1367) (width 0.2) (layer "B.Cu") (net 1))
 (segment (start 77.9605 69.6605) (end 72.1 63.8) (width 0.2) (layer "B.Cu") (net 1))
 (segment (start 77.9605 91.1367) (end 77.9605 69.6605) (width 0.2) (layer "B.Cu") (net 1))
 (segment (start 79.72 63.8) (end 81.29 62.23) (width 0.2) (layer "F.Cu") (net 2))
 (segment (start 81.29 62.23) (end 93.4625 62.23) (width 0.2) (layer "F.Cu") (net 2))
 (segment (start 94.2975 62.23) (end 93.4625 62.23) (width 0.2) (layer "F.Cu") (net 2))
 (segment (start 106.8847 73.0614) (end 106.8847 73.0045) (width 0.2) (layer "F.Cu") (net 21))
 (segment (start 105.0988 71.2755) (end 107.0263 73.2029) (width 0.2) (layer "F.Cu") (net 21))
 (segment (start 107.0263 73.2029) (end 106.8847 73.0614) (width 0.2) (layer "F.Cu") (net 21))
 (segment (start 83.2175 69.0291) (end 85.4639 71.2755) (width 0.2) (layer "F.Cu") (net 21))
 (segment (start 73.7791 69.0291) (end 83.2175 69.0291) (width 0.2) (layer "F.Cu") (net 21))
 (segment (start 85.4639 71.2755) (end 105.0988 71.2755) (width 0.2) (layer "F.Cu") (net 21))
 (segment (start 72.1 67.35) (end 73.7791 69.0291) (width 0.2) (layer "F.Cu") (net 21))
 (via (at 106.8847 73.0045) (size 0.6) (drill 0.3) (layers "F.Cu" "B.Cu") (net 21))
 (segment (start 107.1659 73.3426) (end 106.8847 73.0614) (width 0.2) (layer "B.Cu") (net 21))
 (segment (start 106.8847 73.0614) (end 106.8847 73.0045) (width 0.2) (layer "B.Cu") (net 21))
 (segment (start 107.1659 73.3426) (end 107.1659 82.2421) (width 0.2) (layer "B.Cu") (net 21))
 (segment (start 107.1659 82.2421) (end 108.1088 83.185) (width 0.2) (layer "B.Cu") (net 21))
 (segment (start 78.5849 63.3339) (end 80.3846 61.5342) (width 0.2) (layer "F.Cu") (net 14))
 (segment (start 80.3846 61.5342) (end 91.6183 61.5342) (width 0.2) (layer "F.Cu") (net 14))
 (segment (start 79.72 67.35) (end 78.5849 66.2149) (width 0.2) (layer "F.Cu") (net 14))
 (segment (start 94.2975 59.69) (end 93.4625 59.69) (width 0.2) (layer "F.Cu") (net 14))
 (segment (start 78.5849 66.2149) (end 78.5849 63.3339) (width 0.2) (layer "F.Cu") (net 14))
 (segment (start 91.6183 61.5342) (end 93.4625 59.69) (width 0.2) (layer "F.Cu") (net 14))
 (segment (start 93.4625 57.15) (end 90.1825 60.43) (width 0.2) (layer "F.Cu") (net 13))
 (segment (start 90.1825 60.43) (end 81.3198 60.43) (width 0.2) (layer "F.Cu") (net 13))
 (segment (start 94.2975 57.15) (end 93.4625 57.15) (width 0.2) (layer "F.Cu") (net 13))
 (via (at 81.3198 60.43) (size 0.6) (drill 0.3) (layers "F.Cu" "B.Cu") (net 13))
 (segment (start 81.3198 69.3002) (end 79.72 70.9) (width 0.2) (layer "B.Cu") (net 13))
 (segment (start 81.3198 60.43) (end 81.3198 69.3002) (width 0.2) (layer "B.Cu") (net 13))
 (segment (start 84.8214 73.3426) (end 74.5426 73.3426) (width 0.2) (layer "F.Cu") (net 20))
 (segment (start 74.5426 73.3426) (end 72.1 70.9) (width 0.2) (layer "F.Cu") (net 20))
 (via (at 84.8214 73.3426) (size 0.6) (drill 0.3) (layers "F.Cu" "B.Cu") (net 20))
 (segment (start 89.0588 83.185) (end 89.0588 77.58) (width 0.2) (layer "B.Cu") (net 20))
 (segment (start 89.0588 77.58) (end 84.8214 73.3426) (width 0.2) (layer "B.Cu") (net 20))
 (segment (start 111.9377 70.602) (end 111.4194 71.1203) (width 0.2) (layer "F.Cu") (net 4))
 (segment (start 105.7352 75.63) (end 83.3387 75.63) (width 0.2) (layer "F.Cu") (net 4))
 (segment (start 108.4604 71.9512) (end 108.4604 72.9048) (width 0.2) (layer "F.Cu") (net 4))
 (segment (start 110.3725 67.31) (end 111.9377 68.8752) (width 0.2) (layer "F.Cu") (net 4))
 (segment (start 108.4604 72.9048) (end 105.7352 75.63) (width 0.2) (layer "F.Cu") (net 4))
 (segment (start 83.3387 75.63) (end 70.8625 88.1062) (width 0.2) (layer "F.Cu") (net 4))
 (segment (start 111.4194 71.1203) (end 109.2913 71.1203) (width 0.2) (layer "F.Cu") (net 4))
 (segment (start 109.5375 67.31) (end 110.3725 67.31) (width 0.2) (layer "F.Cu") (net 4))
 (segment (start 70.8625 88.1062) (end 66.4625 88.1062) (width 0.2) (layer "F.Cu") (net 4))
 (segment (start 111.9377 68.8752) (end 111.9377 70.602) (width 0.2) (layer "F.Cu") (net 4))
 (segment (start 109.2913 71.1203) (end 108.4604 71.9512) (width 0.2) (layer "F.Cu") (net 4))
 (segment (start 105.9203 68.3872) (end 85.0688 68.3872) (width 0.2) (layer "F.Cu") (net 6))
 (segment (start 109.5375 64.77) (end 105.9203 68.3872) (width 0.2) (layer "F.Cu") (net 6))
 (segment (start 110.3725 64.77) (end 109.5375 64.77) (width 0.2) (layer "F.Cu") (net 6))
 (segment (start 85.0688 68.3872) (end 84.4853 67.8037) (width 0.2) (layer "F.Cu") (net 6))
 (via (at 84.4853 67.8037) (size 0.6) (drill 0.3) (layers "F.Cu" "B.Cu") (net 6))
 (segment (start 84.2197 68.0693) (end 84.2197 84.849) (width 0.2) (layer "B.Cu") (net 6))
 (segment (start 84.2197 84.849) (end 80.9625 88.1062) (width 0.2) (layer "B.Cu") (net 6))
 (segment (start 84.4853 67.8037) (end 84.2197 68.0693) (width 0.2) (layer "B.Cu") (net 6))
 (segment (start 76.8624 74.008) (end 67.7642 83.1062) (width 0.2) (layer "F.Cu") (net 3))
 (segment (start 106.3805 73.8417) (end 106.2142 74.008) (width 0.2) (layer "F.Cu") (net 3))
 (segment (start 108.0587 71.3288) (end 108.0587 72.7385) (width 0.2) (layer "F.Cu") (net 3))
 (segment (start 66.4625 83.1062) (end 67.7642 83.1062) (width 0.2) (layer "F.Cu") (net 3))
 (segment (start 106.2142 74.008) (end 76.8624 74.008) (width 0.2) (layer "F.Cu") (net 3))
 (segment (start 106.3805 73.8417) (end 106.2142 74.008) (width 0.2) (layer "F.Cu") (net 3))
 (segment (start 109.5375 69.85) (end 110.3725 69.85) (width 0.2) (layer "F.Cu") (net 3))
 (segment (start 109.5375 69.85) (end 108.0587 71.3288) (width 0.2) (layer "F.Cu") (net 3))
 (segment (start 108.0587 72.7385) (end 107.1909 73.6063) (width 0.2) (layer "F.Cu") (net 3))
 (segment (start 106.6159 73.6063) (end 106.3805 73.8417) (width 0.2) (layer "F.Cu") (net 3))
 (segment (start 107.1909 73.6063) (end 106.6159 73.6063) (width 0.2) (layer "F.Cu") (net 3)))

